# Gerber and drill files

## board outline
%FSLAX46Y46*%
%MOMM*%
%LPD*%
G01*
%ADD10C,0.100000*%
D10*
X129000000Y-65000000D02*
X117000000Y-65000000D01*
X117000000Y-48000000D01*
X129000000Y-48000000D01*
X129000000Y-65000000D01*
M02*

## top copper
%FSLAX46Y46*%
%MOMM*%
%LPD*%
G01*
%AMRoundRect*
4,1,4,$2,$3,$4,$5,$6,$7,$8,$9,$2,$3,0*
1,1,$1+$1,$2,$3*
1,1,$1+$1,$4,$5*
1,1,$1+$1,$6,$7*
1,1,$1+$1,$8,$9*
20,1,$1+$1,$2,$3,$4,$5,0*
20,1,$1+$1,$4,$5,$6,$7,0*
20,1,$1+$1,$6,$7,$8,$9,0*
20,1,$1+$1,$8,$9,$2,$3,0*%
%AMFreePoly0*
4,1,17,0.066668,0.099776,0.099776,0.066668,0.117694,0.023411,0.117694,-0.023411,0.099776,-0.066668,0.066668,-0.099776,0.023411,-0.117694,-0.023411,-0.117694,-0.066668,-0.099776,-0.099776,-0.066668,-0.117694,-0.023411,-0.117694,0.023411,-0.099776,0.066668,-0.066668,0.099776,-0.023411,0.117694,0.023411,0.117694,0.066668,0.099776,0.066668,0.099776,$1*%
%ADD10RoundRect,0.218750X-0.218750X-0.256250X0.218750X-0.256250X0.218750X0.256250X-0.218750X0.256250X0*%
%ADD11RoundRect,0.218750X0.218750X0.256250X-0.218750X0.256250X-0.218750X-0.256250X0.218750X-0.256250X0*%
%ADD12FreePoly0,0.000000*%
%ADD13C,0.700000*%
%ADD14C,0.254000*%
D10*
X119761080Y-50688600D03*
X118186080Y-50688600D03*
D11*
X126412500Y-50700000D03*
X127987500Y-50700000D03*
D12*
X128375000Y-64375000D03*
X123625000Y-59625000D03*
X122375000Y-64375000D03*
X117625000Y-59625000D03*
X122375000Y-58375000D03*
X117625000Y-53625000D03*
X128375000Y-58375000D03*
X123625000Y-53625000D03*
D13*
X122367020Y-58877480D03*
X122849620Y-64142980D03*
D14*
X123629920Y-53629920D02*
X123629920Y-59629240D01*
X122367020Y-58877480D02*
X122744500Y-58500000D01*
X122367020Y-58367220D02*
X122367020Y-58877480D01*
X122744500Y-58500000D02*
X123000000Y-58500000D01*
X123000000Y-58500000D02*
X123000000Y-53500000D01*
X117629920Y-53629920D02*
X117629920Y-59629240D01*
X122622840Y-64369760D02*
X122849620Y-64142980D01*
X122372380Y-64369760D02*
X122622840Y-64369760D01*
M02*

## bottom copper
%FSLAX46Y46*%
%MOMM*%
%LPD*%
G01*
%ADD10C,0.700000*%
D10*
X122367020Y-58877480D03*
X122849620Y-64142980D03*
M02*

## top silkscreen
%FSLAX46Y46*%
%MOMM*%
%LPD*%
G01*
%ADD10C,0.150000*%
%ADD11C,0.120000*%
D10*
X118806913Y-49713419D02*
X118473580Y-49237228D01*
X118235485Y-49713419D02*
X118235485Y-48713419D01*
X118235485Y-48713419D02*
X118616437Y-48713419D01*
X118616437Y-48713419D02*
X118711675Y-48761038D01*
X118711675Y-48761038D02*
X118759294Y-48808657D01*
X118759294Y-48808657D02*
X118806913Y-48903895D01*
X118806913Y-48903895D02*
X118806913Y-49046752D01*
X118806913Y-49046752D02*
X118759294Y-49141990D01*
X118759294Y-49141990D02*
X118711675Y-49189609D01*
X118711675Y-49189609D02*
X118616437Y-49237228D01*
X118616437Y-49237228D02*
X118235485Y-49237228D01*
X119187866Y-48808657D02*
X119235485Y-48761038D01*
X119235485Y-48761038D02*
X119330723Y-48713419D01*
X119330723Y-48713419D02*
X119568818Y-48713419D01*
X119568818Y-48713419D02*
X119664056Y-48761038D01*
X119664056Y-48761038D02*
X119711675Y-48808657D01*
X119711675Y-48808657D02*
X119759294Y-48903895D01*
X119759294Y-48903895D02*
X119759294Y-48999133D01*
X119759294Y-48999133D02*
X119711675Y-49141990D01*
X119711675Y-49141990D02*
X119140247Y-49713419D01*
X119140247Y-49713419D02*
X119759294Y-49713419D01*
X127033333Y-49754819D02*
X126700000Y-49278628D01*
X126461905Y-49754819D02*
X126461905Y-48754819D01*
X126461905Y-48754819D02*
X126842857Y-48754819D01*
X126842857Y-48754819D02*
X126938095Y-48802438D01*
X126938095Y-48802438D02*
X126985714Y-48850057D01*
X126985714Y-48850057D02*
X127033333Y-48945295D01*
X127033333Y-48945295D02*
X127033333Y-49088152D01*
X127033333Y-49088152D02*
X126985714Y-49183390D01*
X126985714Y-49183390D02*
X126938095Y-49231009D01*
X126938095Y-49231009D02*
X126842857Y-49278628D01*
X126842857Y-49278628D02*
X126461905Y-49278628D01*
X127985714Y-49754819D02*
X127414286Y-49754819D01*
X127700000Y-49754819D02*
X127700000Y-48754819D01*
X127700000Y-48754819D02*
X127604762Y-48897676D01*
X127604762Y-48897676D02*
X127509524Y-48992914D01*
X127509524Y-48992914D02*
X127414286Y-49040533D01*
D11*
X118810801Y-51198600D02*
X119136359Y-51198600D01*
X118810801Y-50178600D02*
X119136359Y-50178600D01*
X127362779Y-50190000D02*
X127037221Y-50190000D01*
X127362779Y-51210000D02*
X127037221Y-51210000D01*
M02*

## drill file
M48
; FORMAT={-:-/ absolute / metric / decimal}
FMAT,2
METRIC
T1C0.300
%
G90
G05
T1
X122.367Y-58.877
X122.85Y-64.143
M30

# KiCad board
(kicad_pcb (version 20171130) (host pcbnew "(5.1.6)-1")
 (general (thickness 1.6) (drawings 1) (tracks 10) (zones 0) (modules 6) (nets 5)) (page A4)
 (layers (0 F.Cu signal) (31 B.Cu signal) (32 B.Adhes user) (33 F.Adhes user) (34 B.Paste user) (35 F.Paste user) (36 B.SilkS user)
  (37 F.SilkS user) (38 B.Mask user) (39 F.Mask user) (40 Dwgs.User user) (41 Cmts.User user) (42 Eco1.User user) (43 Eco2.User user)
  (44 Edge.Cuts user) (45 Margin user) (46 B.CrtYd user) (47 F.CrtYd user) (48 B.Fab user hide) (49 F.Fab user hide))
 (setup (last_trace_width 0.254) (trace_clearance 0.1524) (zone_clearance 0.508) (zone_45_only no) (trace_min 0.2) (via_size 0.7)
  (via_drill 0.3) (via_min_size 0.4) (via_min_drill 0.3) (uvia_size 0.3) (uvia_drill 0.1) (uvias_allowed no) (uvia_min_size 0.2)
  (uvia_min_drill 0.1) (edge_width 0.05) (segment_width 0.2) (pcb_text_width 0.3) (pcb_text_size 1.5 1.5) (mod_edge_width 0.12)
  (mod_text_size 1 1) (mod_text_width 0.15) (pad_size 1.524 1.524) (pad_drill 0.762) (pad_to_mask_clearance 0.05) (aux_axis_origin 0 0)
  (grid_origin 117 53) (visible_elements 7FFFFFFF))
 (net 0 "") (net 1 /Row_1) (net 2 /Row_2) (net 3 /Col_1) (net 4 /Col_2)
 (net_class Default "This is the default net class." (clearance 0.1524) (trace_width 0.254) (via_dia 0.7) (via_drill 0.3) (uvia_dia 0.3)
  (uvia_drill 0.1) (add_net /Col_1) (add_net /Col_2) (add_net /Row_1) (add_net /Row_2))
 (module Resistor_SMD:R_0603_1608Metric (layer F.Cu) (at 118.97358 50.6886)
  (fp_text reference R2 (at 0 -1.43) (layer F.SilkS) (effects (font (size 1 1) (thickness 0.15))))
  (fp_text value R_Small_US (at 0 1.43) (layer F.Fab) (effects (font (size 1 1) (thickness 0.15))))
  (fp_line (start -0.162779 0.51) (end 0.162779 0.51) (layer F.SilkS) (width 0.12))
  (fp_line (start -0.162779 -0.51) (end 0.162779 -0.51) (layer F.SilkS) (width 0.12))
  (pad 2 smd roundrect (at 0.7875 0) (size 0.875 0.95) (layers F.Cu F.Paste F.Mask) (roundrect_rratio 0.25) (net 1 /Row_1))
  (pad 1 smd roundrect (at -0.7875 0) (size 0.875 0.95) (layers F.Cu F.Paste F.Mask) (roundrect_rratio 0.25) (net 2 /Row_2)))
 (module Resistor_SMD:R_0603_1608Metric (layer F.Cu) (at 127.2 50.7 180)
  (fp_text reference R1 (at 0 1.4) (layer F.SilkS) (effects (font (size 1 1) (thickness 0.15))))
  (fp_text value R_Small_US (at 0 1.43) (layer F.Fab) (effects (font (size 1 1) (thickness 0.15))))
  (fp_line (start -0.162779 0.51) (end 0.162779 0.51) (layer F.SilkS) (width 0.12))
  (fp_line (start -0.162779 -0.51) (end 0.162779 -0.51) (layer F.SilkS) (width 0.12))
  (pad 2 smd roundrect (at 0.7875 0 180) (size 0.875 0.95) (layers F.Cu F.Paste F.Mask) (roundrect_rratio 0.25) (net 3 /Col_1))
  (pad 1 smd roundrect (at -0.7875 0 180) (size 0.875 0.95) (layers F.Cu F.Paste F.Mask) (roundrect_rratio 0.25) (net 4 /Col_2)))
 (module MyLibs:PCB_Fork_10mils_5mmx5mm (layer F.Cu) (at 123.5 59.5)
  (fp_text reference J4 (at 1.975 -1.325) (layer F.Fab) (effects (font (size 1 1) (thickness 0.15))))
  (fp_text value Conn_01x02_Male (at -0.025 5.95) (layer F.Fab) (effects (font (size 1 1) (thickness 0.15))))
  (pad 1 smd custom (at 4.875 4.875) (size 0.24 0.24) (layers F.Cu F.Mask) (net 2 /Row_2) (zone_connect 0)
   (options (clearance outline) (anchor circle)) (primitives))
  (pad 2 smd custom (at 0.125 0.125) (size 0.24 0.24) (layers F.Cu F.Mask) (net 4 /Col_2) (zone_connect 0)
   (options (clearance outline) (anchor circle)) (primitives)))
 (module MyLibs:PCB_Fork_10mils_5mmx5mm (layer F.Cu) (at 117.5 59.5)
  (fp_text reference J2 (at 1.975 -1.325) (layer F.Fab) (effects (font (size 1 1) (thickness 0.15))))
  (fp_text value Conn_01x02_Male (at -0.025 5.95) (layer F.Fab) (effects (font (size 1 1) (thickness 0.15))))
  (pad 1 smd custom (at 4.875 4.875) (size 0.24 0.24) (layers F.Cu F.Mask) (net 2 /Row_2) (zone_connect 0)
   (options (clearance outline) (anchor circle)) (primitives))
  (pad 2 smd custom (at 0.125 0.125) (size 0.24 0.24) (layers F.Cu F.Mask) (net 3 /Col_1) (zone_connect 0)
   (options (clearance outline) (anchor circle)) (primitives)))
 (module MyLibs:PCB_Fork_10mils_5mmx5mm (layer F.Cu) (at 117.5 53.5)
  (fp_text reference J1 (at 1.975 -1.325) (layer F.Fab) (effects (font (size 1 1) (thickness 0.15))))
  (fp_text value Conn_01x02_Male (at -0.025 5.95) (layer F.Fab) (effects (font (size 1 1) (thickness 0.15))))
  (pad 1 smd custom (at 4.875 4.875) (size 0.24 0.24) (layers F.Cu F.Mask) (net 1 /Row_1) (zone_connect 0)
   (options (clearance outline) (anchor circle)) (primitives))
  (pad 2 smd custom (at 0.125 0.125) (size 0.24 0.24) (layers F.Cu F.Mask) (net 3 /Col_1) (zone_connect 0)
   (options (clearance outline) (anchor circle)) (primitives)))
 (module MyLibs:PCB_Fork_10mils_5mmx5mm (layer F.Cu) (at 123.5 53.5)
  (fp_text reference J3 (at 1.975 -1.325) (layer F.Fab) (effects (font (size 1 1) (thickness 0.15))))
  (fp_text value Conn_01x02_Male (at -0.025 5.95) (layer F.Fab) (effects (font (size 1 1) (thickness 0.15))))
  (pad 1 smd custom (at 4.875 4.875) (size 0.24 0.24) (layers F.Cu F.Mask) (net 1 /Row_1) (zone_connect 0)
   (options (clearance outline) (anchor circle)) (primitives))
  (pad 2 smd custom (at 0.125 0.125) (size 0.24 0.24) (layers F.Cu F.Mask) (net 4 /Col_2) (zone_connect 0)
   (options (clearance outline) (anchor circle)) (primitives)))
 (gr_poly (pts (xy 129 65) (xy 117 65) (xy 117 48) (xy 129 48)) (layer Edge.Cuts) (width 0.1))
 (segment (start 123.62992 53.62992) (end 123.62992 59.62924) (width 0.254) (layer F.Cu) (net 4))
 (via (at 122.36702 58.87748) (size 0.7) (drill 0.3) (layers F.Cu B.Cu) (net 1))
 (segment (start 122.36702 58.87748) (end 122.7445 58.5) (width 0.254) (layer F.Cu) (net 1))
 (segment (start 122.36702 58.36722) (end 122.36702 58.87748) (width 0.254) (layer F.Cu) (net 1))
 (segment (start 122.7445 58.5) (end 123 58.5) (width 0.254) (layer F.Cu) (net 1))
 (segment (start 123 58.5) (end 123 53.5) (width 0.254) (layer F.Cu) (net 1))
 (segment (start 117.62992 53.62992) (end 117.62992 59.62924) (width 0.254) (layer F.Cu) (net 3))
 (segment (start 122.62284 64.36976) (end 122.84962 64.14298) (width 0.254) (layer F.Cu) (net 2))
 (segment (start 122.37238 64.36976) (end 122.62284 64.36976) (width 0.254) (layer F.Cu) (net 2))
 (via (at 122.84962 64.14298) (size 0.7) (drill 0.3) (layers F.Cu B.Cu) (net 2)))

